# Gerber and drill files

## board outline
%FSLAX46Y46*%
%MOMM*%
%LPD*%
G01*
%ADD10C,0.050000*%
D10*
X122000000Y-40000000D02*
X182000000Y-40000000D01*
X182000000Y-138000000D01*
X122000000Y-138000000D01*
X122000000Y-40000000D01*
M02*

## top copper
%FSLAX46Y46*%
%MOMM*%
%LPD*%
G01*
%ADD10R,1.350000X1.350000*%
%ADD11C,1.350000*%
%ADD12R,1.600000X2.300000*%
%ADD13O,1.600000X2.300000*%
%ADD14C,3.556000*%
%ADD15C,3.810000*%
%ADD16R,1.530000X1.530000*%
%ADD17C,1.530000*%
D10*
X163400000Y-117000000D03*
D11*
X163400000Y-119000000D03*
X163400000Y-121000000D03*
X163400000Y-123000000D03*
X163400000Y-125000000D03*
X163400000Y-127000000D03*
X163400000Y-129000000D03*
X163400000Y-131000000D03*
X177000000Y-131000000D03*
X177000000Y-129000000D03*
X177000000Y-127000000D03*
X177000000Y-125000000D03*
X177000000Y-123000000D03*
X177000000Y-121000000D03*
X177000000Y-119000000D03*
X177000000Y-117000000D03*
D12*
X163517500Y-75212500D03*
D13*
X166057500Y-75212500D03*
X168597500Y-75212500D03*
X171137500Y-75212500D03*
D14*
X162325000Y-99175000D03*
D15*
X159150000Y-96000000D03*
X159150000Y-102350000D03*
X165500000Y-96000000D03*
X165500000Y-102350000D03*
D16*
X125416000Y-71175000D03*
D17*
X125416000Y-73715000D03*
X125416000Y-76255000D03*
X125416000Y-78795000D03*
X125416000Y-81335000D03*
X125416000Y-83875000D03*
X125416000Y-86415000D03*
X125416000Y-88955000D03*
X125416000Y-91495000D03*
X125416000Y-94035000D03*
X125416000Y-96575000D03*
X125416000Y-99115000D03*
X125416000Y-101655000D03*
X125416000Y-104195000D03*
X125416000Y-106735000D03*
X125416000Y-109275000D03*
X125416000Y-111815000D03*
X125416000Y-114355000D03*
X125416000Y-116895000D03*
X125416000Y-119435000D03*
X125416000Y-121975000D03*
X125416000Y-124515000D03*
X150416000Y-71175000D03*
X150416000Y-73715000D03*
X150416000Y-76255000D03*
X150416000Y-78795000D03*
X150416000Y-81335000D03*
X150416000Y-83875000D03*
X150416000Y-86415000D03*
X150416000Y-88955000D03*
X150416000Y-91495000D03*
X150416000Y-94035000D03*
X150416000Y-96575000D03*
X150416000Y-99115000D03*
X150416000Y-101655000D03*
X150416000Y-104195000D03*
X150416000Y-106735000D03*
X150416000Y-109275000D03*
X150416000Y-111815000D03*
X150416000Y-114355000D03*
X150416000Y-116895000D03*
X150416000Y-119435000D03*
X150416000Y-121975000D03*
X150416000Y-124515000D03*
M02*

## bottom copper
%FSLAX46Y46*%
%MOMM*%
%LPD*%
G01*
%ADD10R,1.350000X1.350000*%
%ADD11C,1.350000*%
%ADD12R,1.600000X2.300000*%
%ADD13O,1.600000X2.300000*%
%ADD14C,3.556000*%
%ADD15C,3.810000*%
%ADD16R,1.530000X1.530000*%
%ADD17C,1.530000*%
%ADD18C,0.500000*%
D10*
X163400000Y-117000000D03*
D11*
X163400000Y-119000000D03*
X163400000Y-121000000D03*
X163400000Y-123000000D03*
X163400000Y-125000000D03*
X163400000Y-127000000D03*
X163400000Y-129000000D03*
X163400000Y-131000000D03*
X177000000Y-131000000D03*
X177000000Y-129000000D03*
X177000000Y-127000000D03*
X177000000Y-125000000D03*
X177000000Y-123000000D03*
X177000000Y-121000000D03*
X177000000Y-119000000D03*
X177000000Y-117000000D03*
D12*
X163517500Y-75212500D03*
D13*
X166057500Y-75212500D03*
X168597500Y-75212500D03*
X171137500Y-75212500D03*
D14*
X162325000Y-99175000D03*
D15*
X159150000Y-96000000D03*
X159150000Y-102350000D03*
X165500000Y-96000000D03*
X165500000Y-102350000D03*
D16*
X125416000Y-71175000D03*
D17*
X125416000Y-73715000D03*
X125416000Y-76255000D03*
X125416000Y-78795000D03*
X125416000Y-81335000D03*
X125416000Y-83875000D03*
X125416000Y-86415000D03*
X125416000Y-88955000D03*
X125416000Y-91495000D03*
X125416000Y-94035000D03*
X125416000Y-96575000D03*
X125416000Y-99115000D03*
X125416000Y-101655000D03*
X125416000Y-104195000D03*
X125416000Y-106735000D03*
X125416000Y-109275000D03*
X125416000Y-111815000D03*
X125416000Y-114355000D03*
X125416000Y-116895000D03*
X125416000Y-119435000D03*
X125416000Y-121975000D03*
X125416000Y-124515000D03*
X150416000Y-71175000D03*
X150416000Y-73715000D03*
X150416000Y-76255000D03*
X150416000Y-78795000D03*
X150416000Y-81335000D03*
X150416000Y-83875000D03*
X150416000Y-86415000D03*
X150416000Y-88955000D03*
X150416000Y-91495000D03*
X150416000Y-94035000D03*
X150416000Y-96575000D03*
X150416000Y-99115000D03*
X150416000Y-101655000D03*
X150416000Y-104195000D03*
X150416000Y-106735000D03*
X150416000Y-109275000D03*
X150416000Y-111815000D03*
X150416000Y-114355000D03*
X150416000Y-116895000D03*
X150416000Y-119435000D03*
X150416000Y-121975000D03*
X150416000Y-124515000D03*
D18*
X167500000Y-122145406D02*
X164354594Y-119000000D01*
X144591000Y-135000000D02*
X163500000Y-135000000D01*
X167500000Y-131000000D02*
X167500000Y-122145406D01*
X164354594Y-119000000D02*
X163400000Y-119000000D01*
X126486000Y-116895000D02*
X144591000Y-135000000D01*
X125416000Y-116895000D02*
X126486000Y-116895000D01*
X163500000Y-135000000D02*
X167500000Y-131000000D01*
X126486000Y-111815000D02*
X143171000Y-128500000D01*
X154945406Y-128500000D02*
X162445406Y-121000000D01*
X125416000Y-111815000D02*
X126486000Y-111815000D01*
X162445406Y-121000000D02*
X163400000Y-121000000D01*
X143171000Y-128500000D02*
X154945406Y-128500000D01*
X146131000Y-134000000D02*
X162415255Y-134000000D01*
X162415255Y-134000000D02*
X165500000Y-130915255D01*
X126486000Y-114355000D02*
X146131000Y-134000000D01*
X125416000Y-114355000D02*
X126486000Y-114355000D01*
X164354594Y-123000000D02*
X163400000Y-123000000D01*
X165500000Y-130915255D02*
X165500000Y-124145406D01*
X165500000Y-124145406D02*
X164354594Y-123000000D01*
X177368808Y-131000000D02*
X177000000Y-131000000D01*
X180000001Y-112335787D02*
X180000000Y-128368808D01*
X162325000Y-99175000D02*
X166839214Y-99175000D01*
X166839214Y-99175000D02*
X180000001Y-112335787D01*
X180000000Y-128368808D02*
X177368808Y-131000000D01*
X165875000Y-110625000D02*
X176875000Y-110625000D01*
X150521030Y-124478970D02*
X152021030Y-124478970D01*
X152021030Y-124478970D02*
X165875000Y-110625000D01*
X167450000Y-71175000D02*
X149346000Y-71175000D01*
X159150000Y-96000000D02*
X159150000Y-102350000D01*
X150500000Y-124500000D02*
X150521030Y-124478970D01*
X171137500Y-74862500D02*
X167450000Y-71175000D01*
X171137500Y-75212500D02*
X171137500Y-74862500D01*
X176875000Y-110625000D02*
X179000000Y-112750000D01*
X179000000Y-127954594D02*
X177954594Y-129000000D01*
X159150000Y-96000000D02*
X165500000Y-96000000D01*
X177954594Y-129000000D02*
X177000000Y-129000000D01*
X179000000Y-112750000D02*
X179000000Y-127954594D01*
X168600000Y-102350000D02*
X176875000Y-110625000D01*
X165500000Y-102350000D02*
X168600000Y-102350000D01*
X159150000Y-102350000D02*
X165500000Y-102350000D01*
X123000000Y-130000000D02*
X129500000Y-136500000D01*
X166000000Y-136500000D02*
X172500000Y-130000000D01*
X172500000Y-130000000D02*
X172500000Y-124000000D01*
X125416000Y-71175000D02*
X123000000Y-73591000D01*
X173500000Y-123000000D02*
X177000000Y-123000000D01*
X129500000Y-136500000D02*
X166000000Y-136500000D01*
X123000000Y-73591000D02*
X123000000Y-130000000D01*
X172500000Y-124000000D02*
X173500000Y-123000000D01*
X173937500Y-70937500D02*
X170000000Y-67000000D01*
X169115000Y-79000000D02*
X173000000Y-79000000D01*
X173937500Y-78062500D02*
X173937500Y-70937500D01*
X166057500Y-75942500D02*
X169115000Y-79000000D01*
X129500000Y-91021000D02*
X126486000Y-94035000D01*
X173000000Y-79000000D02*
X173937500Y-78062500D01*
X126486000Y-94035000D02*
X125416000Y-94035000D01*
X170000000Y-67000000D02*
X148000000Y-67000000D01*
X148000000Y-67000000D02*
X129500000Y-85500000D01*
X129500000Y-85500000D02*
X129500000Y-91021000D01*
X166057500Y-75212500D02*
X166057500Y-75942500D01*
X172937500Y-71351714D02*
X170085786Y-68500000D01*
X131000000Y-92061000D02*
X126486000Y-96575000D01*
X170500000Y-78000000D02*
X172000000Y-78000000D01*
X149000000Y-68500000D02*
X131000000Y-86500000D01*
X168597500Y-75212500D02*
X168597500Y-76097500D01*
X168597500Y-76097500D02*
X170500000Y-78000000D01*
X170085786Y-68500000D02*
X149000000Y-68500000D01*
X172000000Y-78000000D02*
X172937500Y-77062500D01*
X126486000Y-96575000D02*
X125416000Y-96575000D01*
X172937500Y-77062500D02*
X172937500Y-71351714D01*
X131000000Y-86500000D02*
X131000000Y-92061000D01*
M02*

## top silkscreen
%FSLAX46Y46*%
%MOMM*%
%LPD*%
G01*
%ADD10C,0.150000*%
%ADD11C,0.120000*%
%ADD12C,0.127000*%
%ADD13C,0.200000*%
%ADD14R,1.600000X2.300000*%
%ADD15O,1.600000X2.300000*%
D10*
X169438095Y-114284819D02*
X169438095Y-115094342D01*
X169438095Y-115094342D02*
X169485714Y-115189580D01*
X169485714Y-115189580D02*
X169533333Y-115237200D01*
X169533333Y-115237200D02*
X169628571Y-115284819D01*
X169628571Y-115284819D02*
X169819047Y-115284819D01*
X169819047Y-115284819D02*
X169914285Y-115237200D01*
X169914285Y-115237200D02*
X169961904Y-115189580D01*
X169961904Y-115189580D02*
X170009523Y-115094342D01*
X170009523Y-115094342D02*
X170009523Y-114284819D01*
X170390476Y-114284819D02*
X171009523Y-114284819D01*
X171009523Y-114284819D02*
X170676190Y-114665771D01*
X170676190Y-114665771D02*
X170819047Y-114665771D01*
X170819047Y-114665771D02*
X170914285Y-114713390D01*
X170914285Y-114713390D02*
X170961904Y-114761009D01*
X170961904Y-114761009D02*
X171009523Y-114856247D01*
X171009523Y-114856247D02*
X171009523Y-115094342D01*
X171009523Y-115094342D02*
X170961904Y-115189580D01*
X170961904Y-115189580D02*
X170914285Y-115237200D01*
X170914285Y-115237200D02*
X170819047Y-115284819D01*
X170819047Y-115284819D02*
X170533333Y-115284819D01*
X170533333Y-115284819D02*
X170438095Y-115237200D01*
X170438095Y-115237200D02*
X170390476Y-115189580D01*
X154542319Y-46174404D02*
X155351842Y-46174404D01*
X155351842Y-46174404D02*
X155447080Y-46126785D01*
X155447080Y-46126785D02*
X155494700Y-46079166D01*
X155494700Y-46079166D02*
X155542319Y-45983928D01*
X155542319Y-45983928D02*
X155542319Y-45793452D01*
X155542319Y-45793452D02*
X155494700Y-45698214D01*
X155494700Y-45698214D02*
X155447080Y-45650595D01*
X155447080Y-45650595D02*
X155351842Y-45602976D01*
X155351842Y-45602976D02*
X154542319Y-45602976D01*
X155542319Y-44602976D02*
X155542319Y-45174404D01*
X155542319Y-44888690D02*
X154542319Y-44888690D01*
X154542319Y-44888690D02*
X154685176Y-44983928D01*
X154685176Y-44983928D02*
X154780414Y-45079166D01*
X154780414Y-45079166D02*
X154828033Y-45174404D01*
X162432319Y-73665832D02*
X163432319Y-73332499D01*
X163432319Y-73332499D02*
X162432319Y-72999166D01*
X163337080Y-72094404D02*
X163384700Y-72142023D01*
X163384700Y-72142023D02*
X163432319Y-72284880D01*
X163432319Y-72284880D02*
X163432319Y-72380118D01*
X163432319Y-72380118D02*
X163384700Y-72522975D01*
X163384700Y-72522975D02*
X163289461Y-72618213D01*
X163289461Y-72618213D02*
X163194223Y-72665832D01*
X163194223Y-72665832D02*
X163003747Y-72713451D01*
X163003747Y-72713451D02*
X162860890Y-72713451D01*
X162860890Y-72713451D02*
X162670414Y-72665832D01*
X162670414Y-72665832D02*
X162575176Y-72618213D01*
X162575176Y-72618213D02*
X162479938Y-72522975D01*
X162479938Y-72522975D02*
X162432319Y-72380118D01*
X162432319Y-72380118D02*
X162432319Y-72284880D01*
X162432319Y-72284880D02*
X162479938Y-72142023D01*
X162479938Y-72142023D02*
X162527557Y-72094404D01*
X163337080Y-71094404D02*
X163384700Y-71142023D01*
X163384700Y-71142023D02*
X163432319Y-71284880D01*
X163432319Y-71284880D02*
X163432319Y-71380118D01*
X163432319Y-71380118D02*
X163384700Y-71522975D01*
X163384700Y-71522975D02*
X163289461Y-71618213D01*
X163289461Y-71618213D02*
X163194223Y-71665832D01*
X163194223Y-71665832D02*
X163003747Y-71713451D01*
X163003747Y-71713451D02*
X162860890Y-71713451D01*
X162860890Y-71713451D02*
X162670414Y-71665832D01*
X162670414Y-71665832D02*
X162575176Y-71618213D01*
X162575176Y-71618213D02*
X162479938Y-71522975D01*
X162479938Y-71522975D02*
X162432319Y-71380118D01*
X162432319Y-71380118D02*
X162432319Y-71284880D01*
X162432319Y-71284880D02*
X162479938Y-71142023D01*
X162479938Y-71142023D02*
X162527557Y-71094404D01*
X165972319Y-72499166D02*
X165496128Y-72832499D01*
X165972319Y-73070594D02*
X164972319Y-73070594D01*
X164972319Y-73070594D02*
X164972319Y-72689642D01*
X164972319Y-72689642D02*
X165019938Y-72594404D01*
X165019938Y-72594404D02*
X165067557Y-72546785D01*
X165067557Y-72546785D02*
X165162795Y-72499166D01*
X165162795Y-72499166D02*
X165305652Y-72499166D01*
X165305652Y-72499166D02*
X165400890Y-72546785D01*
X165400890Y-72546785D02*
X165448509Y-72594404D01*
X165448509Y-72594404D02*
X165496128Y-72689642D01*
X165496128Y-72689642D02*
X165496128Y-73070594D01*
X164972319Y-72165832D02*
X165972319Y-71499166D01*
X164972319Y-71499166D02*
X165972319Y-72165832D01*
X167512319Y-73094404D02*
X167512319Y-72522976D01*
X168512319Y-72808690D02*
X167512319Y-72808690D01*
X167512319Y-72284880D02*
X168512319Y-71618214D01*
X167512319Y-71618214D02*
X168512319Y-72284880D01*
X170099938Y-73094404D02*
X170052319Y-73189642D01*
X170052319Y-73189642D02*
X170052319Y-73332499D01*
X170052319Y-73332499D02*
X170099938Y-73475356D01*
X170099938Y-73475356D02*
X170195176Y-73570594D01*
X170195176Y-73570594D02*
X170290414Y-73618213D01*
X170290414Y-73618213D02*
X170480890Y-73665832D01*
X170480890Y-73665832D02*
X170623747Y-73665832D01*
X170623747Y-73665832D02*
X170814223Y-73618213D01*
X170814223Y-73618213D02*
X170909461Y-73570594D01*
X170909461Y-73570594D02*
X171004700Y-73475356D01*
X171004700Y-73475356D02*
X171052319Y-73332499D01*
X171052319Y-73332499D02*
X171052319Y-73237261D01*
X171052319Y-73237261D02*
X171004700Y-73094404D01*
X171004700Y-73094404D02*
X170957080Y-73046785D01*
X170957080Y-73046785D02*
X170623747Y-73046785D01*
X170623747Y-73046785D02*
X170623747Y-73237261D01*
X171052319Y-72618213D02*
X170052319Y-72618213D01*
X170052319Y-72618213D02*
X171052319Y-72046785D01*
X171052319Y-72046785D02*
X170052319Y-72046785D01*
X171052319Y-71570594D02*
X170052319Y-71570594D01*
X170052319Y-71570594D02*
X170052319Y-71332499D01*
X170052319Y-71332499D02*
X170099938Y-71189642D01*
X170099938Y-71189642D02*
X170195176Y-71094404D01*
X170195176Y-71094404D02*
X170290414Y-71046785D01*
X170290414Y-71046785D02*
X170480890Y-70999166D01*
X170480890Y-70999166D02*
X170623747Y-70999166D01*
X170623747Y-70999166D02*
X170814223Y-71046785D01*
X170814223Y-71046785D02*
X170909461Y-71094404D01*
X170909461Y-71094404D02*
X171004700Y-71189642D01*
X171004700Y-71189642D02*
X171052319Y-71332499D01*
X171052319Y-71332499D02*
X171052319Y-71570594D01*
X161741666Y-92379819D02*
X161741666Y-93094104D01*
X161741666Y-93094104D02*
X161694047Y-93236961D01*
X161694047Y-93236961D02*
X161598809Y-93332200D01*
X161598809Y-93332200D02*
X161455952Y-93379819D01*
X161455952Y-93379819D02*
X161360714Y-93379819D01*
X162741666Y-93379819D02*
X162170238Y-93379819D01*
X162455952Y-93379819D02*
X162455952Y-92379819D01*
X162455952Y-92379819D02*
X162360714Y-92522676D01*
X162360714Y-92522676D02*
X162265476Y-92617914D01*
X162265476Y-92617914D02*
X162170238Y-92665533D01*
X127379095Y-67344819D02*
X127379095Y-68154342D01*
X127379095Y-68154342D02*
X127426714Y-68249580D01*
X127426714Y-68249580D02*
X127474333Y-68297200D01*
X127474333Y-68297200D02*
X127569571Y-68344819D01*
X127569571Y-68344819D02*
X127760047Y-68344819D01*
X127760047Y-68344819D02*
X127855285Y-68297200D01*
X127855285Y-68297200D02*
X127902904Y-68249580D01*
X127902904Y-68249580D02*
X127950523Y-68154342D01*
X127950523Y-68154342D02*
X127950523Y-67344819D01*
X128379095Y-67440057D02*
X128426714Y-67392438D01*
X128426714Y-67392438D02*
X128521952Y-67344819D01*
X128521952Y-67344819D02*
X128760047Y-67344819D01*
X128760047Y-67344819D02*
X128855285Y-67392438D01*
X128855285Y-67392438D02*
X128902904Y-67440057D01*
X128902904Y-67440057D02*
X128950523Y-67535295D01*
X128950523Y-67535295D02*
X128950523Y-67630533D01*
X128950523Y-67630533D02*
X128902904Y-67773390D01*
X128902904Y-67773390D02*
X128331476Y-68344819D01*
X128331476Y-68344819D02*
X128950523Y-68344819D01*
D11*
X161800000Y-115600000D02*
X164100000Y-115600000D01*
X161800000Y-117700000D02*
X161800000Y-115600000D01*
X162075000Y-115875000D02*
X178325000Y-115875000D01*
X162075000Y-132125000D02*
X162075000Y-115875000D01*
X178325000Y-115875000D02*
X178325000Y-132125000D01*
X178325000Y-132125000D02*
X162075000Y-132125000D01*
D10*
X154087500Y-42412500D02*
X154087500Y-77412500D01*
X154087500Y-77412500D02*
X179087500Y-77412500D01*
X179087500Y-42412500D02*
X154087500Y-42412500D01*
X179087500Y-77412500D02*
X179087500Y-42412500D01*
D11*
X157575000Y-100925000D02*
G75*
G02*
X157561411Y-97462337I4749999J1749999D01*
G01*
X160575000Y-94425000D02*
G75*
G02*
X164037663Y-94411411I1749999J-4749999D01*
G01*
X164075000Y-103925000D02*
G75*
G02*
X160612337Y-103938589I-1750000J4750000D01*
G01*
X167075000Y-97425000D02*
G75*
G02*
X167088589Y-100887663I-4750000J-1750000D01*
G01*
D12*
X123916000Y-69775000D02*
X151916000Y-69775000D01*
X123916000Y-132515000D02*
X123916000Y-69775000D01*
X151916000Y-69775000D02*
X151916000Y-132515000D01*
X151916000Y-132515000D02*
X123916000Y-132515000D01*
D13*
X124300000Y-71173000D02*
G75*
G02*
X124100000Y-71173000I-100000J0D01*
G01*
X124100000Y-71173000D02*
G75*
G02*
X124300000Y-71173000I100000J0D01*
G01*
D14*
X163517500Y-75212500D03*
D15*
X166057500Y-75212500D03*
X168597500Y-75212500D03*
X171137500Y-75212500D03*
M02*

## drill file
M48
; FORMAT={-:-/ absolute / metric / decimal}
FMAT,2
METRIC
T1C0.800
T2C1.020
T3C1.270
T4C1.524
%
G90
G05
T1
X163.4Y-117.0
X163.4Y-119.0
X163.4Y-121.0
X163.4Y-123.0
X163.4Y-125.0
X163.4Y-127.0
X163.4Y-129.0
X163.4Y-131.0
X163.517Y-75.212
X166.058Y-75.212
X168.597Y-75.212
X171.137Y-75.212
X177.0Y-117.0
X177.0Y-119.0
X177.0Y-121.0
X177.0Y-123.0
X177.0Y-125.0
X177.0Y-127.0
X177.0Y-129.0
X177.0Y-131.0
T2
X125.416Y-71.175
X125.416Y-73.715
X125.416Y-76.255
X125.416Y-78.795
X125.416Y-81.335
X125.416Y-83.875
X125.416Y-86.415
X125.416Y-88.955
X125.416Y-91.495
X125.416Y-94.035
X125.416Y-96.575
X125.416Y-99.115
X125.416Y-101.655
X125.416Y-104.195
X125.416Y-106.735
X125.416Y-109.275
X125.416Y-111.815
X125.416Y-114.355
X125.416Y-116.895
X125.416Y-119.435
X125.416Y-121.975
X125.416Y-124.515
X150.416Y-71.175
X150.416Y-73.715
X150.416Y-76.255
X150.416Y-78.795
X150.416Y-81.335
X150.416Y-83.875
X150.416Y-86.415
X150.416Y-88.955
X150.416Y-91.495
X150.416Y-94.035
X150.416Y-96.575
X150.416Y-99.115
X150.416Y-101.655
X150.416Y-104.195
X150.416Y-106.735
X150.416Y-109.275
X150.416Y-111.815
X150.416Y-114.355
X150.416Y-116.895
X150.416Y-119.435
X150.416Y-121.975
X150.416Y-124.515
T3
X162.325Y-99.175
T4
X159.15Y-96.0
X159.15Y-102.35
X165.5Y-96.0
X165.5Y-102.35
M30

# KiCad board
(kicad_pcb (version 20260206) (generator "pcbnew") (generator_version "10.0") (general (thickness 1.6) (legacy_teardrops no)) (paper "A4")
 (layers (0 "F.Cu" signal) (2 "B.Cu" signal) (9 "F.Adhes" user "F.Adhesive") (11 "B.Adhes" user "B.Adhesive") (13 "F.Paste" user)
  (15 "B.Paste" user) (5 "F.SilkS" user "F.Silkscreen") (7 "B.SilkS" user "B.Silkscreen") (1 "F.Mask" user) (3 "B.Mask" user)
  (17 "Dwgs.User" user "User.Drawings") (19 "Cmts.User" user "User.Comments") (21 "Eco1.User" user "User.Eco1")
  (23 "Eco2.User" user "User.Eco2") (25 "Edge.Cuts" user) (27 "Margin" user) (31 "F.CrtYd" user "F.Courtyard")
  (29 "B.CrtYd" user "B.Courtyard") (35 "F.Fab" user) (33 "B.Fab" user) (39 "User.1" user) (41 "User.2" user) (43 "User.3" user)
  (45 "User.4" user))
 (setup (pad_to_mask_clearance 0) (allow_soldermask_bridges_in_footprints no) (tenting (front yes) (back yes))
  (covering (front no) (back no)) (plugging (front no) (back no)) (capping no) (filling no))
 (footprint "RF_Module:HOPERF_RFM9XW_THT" (layer "F.Cu") (at 163.4 117)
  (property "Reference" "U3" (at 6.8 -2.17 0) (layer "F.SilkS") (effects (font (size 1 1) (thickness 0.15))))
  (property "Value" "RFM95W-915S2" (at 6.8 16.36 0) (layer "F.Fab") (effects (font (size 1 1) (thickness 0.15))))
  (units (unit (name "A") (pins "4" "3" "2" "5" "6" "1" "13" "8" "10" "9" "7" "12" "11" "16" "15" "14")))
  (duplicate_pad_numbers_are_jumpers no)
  (fp_line (start -1.6 -1.4) (end 0.7 -1.4) (stroke (width 0.12) (type solid)) (layer "F.SilkS"))
  (fp_line (start -1.6 0.7) (end -1.6 -1.4) (stroke (width 0.12) (type solid)) (layer "F.SilkS"))
  (fp_line (start -1.325 -1.125) (end 14.925 -1.125) (stroke (width 0.12) (type solid)) (layer "F.SilkS"))
  (fp_line (start -1.325 15.125) (end -1.325 -1.125) (stroke (width 0.12) (type solid)) (layer "F.SilkS"))
  (fp_line (start 14.925 -1.125) (end 14.925 15.125) (stroke (width 0.12) (type solid)) (layer "F.SilkS"))
  (fp_line (start 14.925 15.125) (end -1.325 15.125) (stroke (width 0.12) (type solid)) (layer "F.SilkS"))
  (pad "1" thru_hole rect (at 0 0) (size 1.35 1.35) (drill 0.8) (layers "*.Cu" "*.Mask") (remove_unused_layers no)
   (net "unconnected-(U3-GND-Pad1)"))
  (pad "2" thru_hole circle (at 0 2) (size 1.35 1.35) (drill 0.8) (layers "*.Cu" "*.Mask") (remove_unused_layers no) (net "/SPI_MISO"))
  (pad "3" thru_hole circle (at 0 4) (size 1.35 1.35) (drill 0.8) (layers "*.Cu" "*.Mask") (remove_unused_layers no) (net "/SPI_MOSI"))
  (pad "4" thru_hole circle (at 0 6) (size 1.35 1.35) (drill 0.8) (layers "*.Cu" "*.Mask") (remove_unused_layers no) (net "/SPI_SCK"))
  (pad "5" thru_hole circle (at 0 8) (size 1.35 1.35) (drill 0.8) (layers "*.Cu" "*.Mask") (remove_unused_layers no) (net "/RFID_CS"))
  (pad "6" thru_hole circle (at 0 10) (size 1.35 1.35) (drill 0.8) (layers "*.Cu" "*.Mask") (remove_unused_layers no) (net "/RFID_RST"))
  (pad "7" thru_hole circle (at 0 12) (size 1.35 1.35) (drill 0.8) (layers "*.Cu" "*.Mask") (remove_unused_layers no)
   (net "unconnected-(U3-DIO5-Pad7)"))
  (pad "8" thru_hole circle (at 0 14) (size 1.35 1.35) (drill 0.8) (layers "*.Cu" "*.Mask") (remove_unused_layers no)
   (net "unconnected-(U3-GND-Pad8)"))
  (pad "9" thru_hole circle (at 13.6 14) (size 1.35 1.35) (drill 0.8) (layers "*.Cu" "*.Mask") (remove_unused_layers no) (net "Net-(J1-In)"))
  (pad "10" thru_hole circle (at 13.6 12) (size 1.35 1.35) (drill 0.8) (layers "*.Cu" "*.Mask") (remove_unused_layers no)
   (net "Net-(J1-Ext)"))
  (pad "11" thru_hole circle (at 13.6 10) (size 1.35 1.35) (drill 0.8) (layers "*.Cu" "*.Mask") (remove_unused_layers no)
   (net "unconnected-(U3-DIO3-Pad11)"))
  (pad "12" thru_hole circle (at 13.6 8) (size 1.35 1.35) (drill 0.8) (layers "*.Cu" "*.Mask") (remove_unused_layers no)
   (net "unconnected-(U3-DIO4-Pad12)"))
  (pad "13" thru_hole circle (at 13.6 6) (size 1.35 1.35) (drill 0.8) (layers "*.Cu" "*.Mask") (remove_unused_layers no)
   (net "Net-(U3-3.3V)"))
  (pad "14" thru_hole circle (at 13.6 4) (size 1.35 1.35) (drill 0.8) (layers "*.Cu" "*.Mask") (remove_unused_layers no)
   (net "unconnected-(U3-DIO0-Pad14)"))
  (pad "15" thru_hole circle (at 13.6 2) (size 1.35 1.35) (drill 0.8) (layers "*.Cu" "*.Mask") (remove_unused_layers no)
   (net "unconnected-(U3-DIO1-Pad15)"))
  (pad "16" thru_hole circle (at 13.6 0) (size 1.35 1.35) (drill 0.8) (layers "*.Cu" "*.Mask") (remove_unused_layers no)
   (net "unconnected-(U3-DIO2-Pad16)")))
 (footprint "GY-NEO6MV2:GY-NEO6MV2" (layer "F.Cu") (at 154.0875 77.4125 -90)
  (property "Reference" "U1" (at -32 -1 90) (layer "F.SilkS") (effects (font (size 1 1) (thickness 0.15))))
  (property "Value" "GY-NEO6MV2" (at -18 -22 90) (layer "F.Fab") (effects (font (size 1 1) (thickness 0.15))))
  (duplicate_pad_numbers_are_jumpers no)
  (fp_line (start -35 0) (end 0 0) (stroke (width 0.15) (type solid)) (layer "F.SilkS"))
  (fp_line (start 0 0) (end 0 -25) (stroke (width 0.15) (type solid)) (layer "F.SilkS"))
  (fp_line (start -35 -25) (end -35 0) (stroke (width 0.15) (type solid)) (layer "F.SilkS"))
  (fp_line (start 0 -25) (end -35 -25) (stroke (width 0.15) (type solid)) (layer "F.SilkS"))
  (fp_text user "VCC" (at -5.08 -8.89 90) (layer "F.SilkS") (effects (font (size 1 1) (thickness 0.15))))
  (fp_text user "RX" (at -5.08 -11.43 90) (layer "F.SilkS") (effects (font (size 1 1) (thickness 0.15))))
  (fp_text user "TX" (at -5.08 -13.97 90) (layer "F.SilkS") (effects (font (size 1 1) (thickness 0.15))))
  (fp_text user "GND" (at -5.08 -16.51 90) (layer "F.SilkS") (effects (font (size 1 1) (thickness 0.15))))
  (pad "1" thru_hole rect (at -2.2 -9.43 270) (size 2.3 1.6) (drill 0.8) (layers "*.Cu" "*.Mask" "F.SilkS") (remove_unused_layers no)
   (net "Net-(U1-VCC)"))
  (pad "2" thru_hole oval (at -2.2 -11.97 270) (size 2.3 1.6) (drill 0.8) (layers "*.Cu" "*.Mask" "F.SilkS") (remove_unused_layers no)
   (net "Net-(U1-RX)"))
  (pad "3" thru_hole oval (at -2.2 -14.51 270) (size 2.3 1.6) (drill 0.8) (layers "*.Cu" "*.Mask" "F.SilkS") (remove_unused_layers no)
   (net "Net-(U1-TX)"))
  (pad "4" thru_hole oval (at -2.2 -17.05 270) (size 2.3 1.6) (drill 0.8) (layers "*.Cu" "*.Mask" "F.SilkS") (remove_unused_layers no)
   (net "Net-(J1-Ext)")))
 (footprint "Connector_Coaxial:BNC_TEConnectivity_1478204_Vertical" (layer "F.Cu") (at 162.325 99.175)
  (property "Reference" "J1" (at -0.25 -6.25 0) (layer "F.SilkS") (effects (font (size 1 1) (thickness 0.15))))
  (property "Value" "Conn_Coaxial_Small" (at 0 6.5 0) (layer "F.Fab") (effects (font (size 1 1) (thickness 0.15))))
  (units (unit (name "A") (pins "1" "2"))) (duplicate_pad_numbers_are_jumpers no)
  (fp_arc (start -4.75 1.75) (mid -5.062075 0.019867) (end -4.763589 -1.712663) (stroke (width 0.12) (type solid)) (layer "F.SilkS"))
  (fp_arc (start -1.75 -4.75) (mid -0.019867 -5.062075) (end 1.712663 -4.763589) (stroke (width 0.12) (type solid)) (layer "F.SilkS"))
  (fp_arc (start 1.75 4.75) (mid 0.019867 5.062075) (end -1.712663 4.763589) (stroke (width 0.12) (type solid)) (layer "F.SilkS"))
  (fp_arc (start 4.75 -1.75) (mid 5.062075 -0.019867) (end 4.763589 1.712663) (stroke (width 0.12) (type solid)) (layer "F.SilkS"))
  (pad "1" thru_hole circle (at 0 0) (size 3.556 3.556) (drill 1.27) (layers "*.Cu" "*.Mask") (remove_unused_layers no) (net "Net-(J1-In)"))
  (pad "2" thru_hole circle (at -3.175 -3.175) (size 3.81 3.81) (drill 1.524) (layers "*.Cu" "*.Mask") (remove_unused_layers no)
   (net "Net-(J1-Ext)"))
  (pad "2" thru_hole circle (at -3.175 3.175) (size 3.81 3.81) (drill 1.524) (layers "*.Cu" "*.Mask") (remove_unused_layers no)
   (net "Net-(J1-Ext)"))
  (pad "2" thru_hole circle (at 3.175 -3.175) (size 3.81 3.81) (drill 1.524) (layers "*.Cu" "*.Mask") (remove_unused_layers no)
   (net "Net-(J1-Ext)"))
  (pad "2" thru_hole circle (at 3.175 3.175) (size 3.81 3.81) (drill 1.524) (layers "*.Cu" "*.Mask") (remove_unused_layers no)
   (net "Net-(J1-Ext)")))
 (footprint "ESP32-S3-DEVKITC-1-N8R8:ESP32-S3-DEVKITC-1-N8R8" (layer "F.Cu") (at 137.916 101.145)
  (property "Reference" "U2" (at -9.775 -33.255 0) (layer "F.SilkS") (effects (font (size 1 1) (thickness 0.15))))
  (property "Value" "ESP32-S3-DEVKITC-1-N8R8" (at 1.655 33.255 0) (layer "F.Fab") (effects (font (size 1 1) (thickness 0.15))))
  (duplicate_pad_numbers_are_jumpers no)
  (fp_line (start -14 -31.37) (end 14 -31.37) (stroke (width 0.127) (type solid)) (layer "F.SilkS"))
  (fp_line (start -14 31.37) (end -14 -31.37) (stroke (width 0.127) (type solid)) (layer "F.SilkS"))
  (fp_line (start 14 -31.37) (end 14 31.37) (stroke (width 0.127) (type solid)) (layer "F.SilkS"))
  (fp_line (start 14 31.37) (end -14 31.37) (stroke (width 0.127) (type solid)) (layer "F.SilkS"))
  (fp_circle (center -13.716 -29.972) (end -13.616 -29.972) (stroke (width 0.2) (type solid)) (fill no) (layer "F.SilkS"))
  (pad "J1_1" thru_hole rect (at -12.5 -29.97) (size 1.53 1.53) (drill 1.02) (layers "*.Cu" "*.Mask") (remove_unused_layers no)
   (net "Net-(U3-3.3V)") (solder_mask_margin 0.102))
  (pad "J1_2" thru_hole circle (at -12.5 -27.43) (size 1.53 1.53) (drill 1.02) (layers "*.Cu" "*.Mask") (remove_unused_layers no)
   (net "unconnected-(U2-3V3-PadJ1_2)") (solder_mask_margin 0.102))
  (pad "J1_3" thru_hole circle (at -12.5 -24.89) (size 1.53 1.53) (drill 1.02) (layers "*.Cu" "*.Mask") (remove_unused_layers no)
   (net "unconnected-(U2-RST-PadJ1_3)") (solder_mask_margin 0.102))
  (pad "J1_4" thru_hole circle (at -12.5 -22.35) (size 1.53 1.53) (drill 1.02) (layers "*.Cu" "*.Mask") (remove_unused_layers no)
   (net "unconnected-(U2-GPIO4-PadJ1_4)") (solder_mask_margin 0.102))
  (pad "J1_5" thru_hole circle (at -12.5 -19.81) (size 1.53 1.53) (drill 1.02) (layers "*.Cu" "*.Mask") (remove_unused_layers no)
   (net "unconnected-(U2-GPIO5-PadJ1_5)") (solder_mask_margin 0.102))
  (pad "J1_6" thru_hole circle (at -12.5 -17.27) (size 1.53 1.53) (drill 1.02) (layers "*.Cu" "*.Mask") (remove_unused_layers no)
   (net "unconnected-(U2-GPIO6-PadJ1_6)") (solder_mask_margin 0.102))
  (pad "J1_7" thru_hole circle (at -12.5 -14.73) (size 1.53 1.53) (drill 1.02) (layers "*.Cu" "*.Mask") (remove_unused_layers no)
   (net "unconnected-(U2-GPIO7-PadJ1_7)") (solder_mask_margin 0.102))
  (pad "J1_8" thru_hole circle (at -12.5 -12.19) (size 1.53 1.53) (drill 1.02) (layers "*.Cu" "*.Mask") (remove_unused_layers no)
   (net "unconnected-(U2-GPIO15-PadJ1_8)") (solder_mask_margin 0.102))
  (pad "J1_9" thru_hole circle (at -12.5 -9.65) (size 1.53 1.53) (drill 1.02) (layers "*.Cu" "*.Mask") (remove_unused_layers no)
   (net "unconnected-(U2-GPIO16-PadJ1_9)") (solder_mask_margin 0.102))
  (pad "J1_10" thru_hole circle (at -12.5 -7.11) (size 1.53 1.53) (drill 1.02) (layers "*.Cu" "*.Mask") (remove_unused_layers no)
   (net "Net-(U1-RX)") (solder_mask_margin 0.102))
  (pad "J1_11" thru_hole circle (at -12.5 -4.57) (size 1.53 1.53) (drill 1.02) (layers "*.Cu" "*.Mask") (remove_unused_layers no)
   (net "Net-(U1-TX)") (solder_mask_margin 0.102))
  (pad "J1_12" thru_hole circle (at -12.5 -2.03) (size 1.53 1.53) (drill 1.02) (layers "*.Cu" "*.Mask") (remove_unused_layers no)
   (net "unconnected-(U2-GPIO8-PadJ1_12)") (solder_mask_margin 0.102))
  (pad "J1_13" thru_hole circle (at -12.5 0.51) (size 1.53 1.53) (drill 1.02) (layers "*.Cu" "*.Mask") (remove_unused_layers no)
   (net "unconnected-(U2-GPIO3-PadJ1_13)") (solder_mask_margin 0.102))
  (pad "J1_14" thru_hole circle (at -12.5 3.05) (size 1.53 1.53) (drill 1.02) (layers "*.Cu" "*.Mask") (remove_unused_layers no)
   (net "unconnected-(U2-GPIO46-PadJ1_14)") (solder_mask_margin 0.102))
  (pad "J1_15" thru_hole circle (at -12.5 5.59) (size 1.53 1.53) (drill 1.02) (layers "*.Cu" "*.Mask") (remove_unused_layers no)
   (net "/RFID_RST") (solder_mask_margin 0.102))
  (pad "J1_16" thru_hole circle (at -12.5 8.13) (size 1.53 1.53) (drill 1.02) (layers "*.Cu" "*.Mask") (remove_unused_layers no)
   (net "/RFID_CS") (solder_mask_margin 0.102))
  (pad "J1_17" thru_hole circle (at -12.5 10.67) (size 1.53 1.53) (drill 1.02) (layers "*.Cu" "*.Mask") (remove_unused_layers no)
   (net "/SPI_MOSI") (solder_mask_margin 0.102))
  (pad "J1_18" thru_hole circle (at -12.5 13.21) (size 1.53 1.53) (drill 1.02) (layers "*.Cu" "*.Mask") (remove_unused_layers no)
   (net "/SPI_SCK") (solder_mask_margin 0.102))
  (pad "J1_19" thru_hole circle (at -12.5 15.75) (size 1.53 1.53) (drill 1.02) (layers "*.Cu" "*.Mask") (remove_unused_layers no)
   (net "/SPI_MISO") (solder_mask_margin 0.102))
  (pad "J1_20" thru_hole circle (at -12.5 18.29) (size 1.53 1.53) (drill 1.02) (layers "*.Cu" "*.Mask") (remove_unused_layers no)
   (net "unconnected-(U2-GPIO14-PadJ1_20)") (solder_mask_margin 0.102))
  (pad "J1_21" thru_hole circle (at -12.5 20.83) (size 1.53 1.53) (drill 1.02) (layers "*.Cu" "*.Mask") (remove_unused_layers no)
   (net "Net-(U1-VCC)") (solder_mask_margin 0.102))
  (pad "J1_22" thru_hole circle (at -12.5 23.37) (size 1.53 1.53) (drill 1.02) (layers "*.Cu" "*.Mask") (remove_unused_layers no)
   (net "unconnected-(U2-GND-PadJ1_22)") (solder_mask_margin 0.102))
  (pad "J3_1" thru_hole circle (at 12.5 -29.97) (size 1.53 1.53) (drill 1.02) (layers "*.Cu" "*.Mask") (remove_unused_layers no)
   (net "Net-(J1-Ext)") (solder_mask_margin 0.102))
  (pad "J3_2" thru_hole circle (at 12.5 -27.43) (size 1.53 1.53) (drill 1.02) (layers "*.Cu" "*.Mask") (remove_unused_layers no)
   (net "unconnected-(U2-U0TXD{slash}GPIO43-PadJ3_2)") (solder_mask_margin 0.102))
  (pad "J3_3" thru_hole circle (at 12.5 -24.89) (size 1.53 1.53) (drill 1.02) (layers "*.Cu" "*.Mask") (remove_unused_layers no)
   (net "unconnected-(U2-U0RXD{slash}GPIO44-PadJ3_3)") (solder_mask_margin 0.102))
  (pad "J3_4" thru_hole circle (at 12.5 -22.35) (size 1.53 1.53) (drill 1.02) (layers "*.Cu" "*.Mask") (remove_unused_layers no)
   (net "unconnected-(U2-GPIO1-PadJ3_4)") (solder_mask_margin 0.102))
  (pad "J3_5" thru_hole circle (at 12.5 -19.81) (size 1.53 1.53) (drill 1.02) (layers "*.Cu" "*.Mask") (remove_unused_layers no)
   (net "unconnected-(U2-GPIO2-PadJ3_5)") (solder_mask_margin 0.102))
  (pad "J3_6" thru_hole circle (at 12.5 -17.27) (size 1.53 1.53) (drill 1.02) (layers "*.Cu" "*.Mask") (remove_unused_layers no)
   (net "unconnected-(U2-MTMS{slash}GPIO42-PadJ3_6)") (solder_mask_margin 0.102))
  (pad "J3_7" thru_hole circle (at 12.5 -14.73) (size 1.53 1.53) (drill 1.02) (layers "*.Cu" "*.Mask") (remove_unused_layers no)
   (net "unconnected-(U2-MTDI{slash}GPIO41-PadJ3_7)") (solder_mask_margin 0.102))
  (pad "J3_8" thru_hole circle (at 12.5 -12.19) (size 1.53 1.53) (drill 1.02) (layers "*.Cu" "*.Mask") (remove_unused_layers no)
   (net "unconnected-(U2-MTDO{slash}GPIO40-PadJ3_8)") (solder_mask_margin 0.102))
  (pad "J3_9" thru_hole circle (at 12.5 -9.65) (size 1.53 1.53) (drill 1.02) (layers "*.Cu" "*.Mask") (remove_unused_layers no)
   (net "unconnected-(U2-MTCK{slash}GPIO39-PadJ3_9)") (solder_mask_margin 0.102))
  (pad "J3_10" thru_hole circle (at 12.5 -7.11) (size 1.53 1.53) (drill 1.02) (layers "*.Cu" "*.Mask") (remove_unused_layers no)
   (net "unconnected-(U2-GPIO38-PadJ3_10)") (solder_mask_margin 0.102))
  (pad "J3_11" thru_hole circle (at 12.5 -4.57) (size 1.53 1.53) (drill 1.02) (layers "*.Cu" "*.Mask") (remove_unused_layers no)
   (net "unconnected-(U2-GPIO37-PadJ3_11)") (solder_mask_margin 0.102))
  (pad "J3_12" thru_hole circle (at 12.5 -2.03) (size 1.53 1.53) (drill 1.02) (layers "*.Cu" "*.Mask") (remove_unused_layers no)
   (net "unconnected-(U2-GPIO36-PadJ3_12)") (solder_mask_margin 0.102))
  (pad "J3_13" thru_hole circle (at 12.5 0.51) (size 1.53 1.53) (drill 1.02) (layers "*.Cu" "*.Mask") (remove_unused_layers no)
   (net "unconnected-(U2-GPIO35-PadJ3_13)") (solder_mask_margin 0.102))
  (pad "J3_14" thru_hole circle (at 12.5 3.05) (size 1.53 1.53) (drill 1.02) (layers "*.Cu" "*.Mask") (remove_unused_layers no)
   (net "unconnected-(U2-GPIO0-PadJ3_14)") (solder_mask_margin 0.102))
  (pad "J3_15" thru_hole circle (at 12.5 5.59) (size 1.53 1.53) (drill 1.02) (layers "*.Cu" "*.Mask") (remove_unused_layers no)
   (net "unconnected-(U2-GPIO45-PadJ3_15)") (solder_mask_margin 0.102))
  (pad "J3_16" thru_hole circle (at 12.5 8.13) (size 1.53 1.53) (drill 1.02) (layers "*.Cu" "*.Mask") (remove_unused_layers no)
   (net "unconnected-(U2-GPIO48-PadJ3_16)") (solder_mask_margin 0.102))
  (pad "J3_17" thru_hole circle (at 12.5 10.67) (size 1.53 1.53) (drill 1.02) (layers "*.Cu" "*.Mask") (remove_unused_layers no)
   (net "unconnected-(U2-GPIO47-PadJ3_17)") (solder_mask_margin 0.102))
  (pad "J3_18" thru_hole circle (at 12.5 13.21) (size 1.53 1.53) (drill 1.02) (layers "*.Cu" "*.Mask") (remove_unused_layers no)
   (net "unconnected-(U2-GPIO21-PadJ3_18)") (solder_mask_margin 0.102))
  (pad "J3_19" thru_hole circle (at 12.5 15.75) (size 1.53 1.53) (drill 1.02) (layers "*.Cu" "*.Mask") (remove_unused_layers no)
   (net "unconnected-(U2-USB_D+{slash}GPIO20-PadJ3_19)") (solder_mask_margin 0.102))
  (pad "J3_20" thru_hole circle (at 12.5 18.29) (size 1.53 1.53) (drill 1.02) (layers "*.Cu" "*.Mask") (remove_unused_layers no)
   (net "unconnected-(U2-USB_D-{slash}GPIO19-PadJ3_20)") (solder_mask_margin 0.102))
  (pad "J3_21" thru_hole circle (at 12.5 20.83) (size 1.53 1.53) (drill 1.02) (layers "*.Cu" "*.Mask") (remove_unused_layers no)
   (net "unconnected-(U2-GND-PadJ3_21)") (solder_mask_margin 0.102))
  (pad "J3_22" thru_hole circle (at 12.5 23.37) (size 1.53 1.53) (drill 1.02) (layers "*.Cu" "*.Mask") (remove_unused_layers no)
   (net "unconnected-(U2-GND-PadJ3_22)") (solder_mask_margin 0.102)))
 (gr_rect (start 122 40) (end 182 138) (stroke (width 0.05) (type solid)) (fill no) (layer "Edge.Cuts"))
 (segment (start 167.5 122.145406) (end 164.354594 119) (width 0.5) (layer "B.Cu") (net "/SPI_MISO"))
 (segment (start 144.591 135) (end 163.5 135) (width 0.5) (layer "B.Cu") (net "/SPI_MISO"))
 (segment (start 167.5 131) (end 167.5 122.145406) (width 0.5) (layer "B.Cu") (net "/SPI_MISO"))
 (segment (start 164.354594 119) (end 163.4 119) (width 0.5) (layer "B.Cu") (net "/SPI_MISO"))
 (segment (start 126.486 116.895) (end 144.591 135) (width 0.5) (layer "B.Cu") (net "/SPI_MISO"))
 (segment (start 125.416 116.895) (end 126.486 116.895) (width 0.5) (layer "B.Cu") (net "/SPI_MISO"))
 (segment (start 163.5 135) (end 167.5 131) (width 0.5) (layer "B.Cu") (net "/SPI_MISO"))
 (segment (start 126.486 111.815) (end 143.171 128.5) (width 0.5) (layer "B.Cu") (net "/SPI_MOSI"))
 (segment (start 154.945406 128.5) (end 162.445406 121) (width 0.5) (layer "B.Cu") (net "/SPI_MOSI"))
 (segment (start 125.416 111.815) (end 126.486 111.815) (width 0.5) (layer "B.Cu") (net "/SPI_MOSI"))
 (segment (start 162.445406 121) (end 163.4 121) (width 0.5) (layer "B.Cu") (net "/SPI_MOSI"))
 (segment (start 143.171 128.5) (end 154.945406 128.5) (width 0.5) (layer "B.Cu") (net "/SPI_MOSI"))
 (segment (start 146.131 134) (end 162.415255 134) (width 0.5) (layer "B.Cu") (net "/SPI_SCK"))
 (segment (start 162.415255 134) (end 165.5 130.915255) (width 0.5) (layer "B.Cu") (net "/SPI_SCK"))
 (segment (start 126.486 114.355) (end 146.131 134) (width 0.5) (layer "B.Cu") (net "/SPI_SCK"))
 (segment (start 125.416 114.355) (end 126.486 114.355) (width 0.5) (layer "B.Cu") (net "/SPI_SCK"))
 (segment (start 164.354594 123) (end 163.4 123) (width 0.5) (layer "B.Cu") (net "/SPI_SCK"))
 (segment (start 165.5 130.915255) (end 165.5 124.145406) (width 0.5) (layer "B.Cu") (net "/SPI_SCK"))
 (segment (start 165.5 124.145406) (end 164.354594 123) (width 0.5) (layer "B.Cu") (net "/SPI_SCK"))
 (segment (start 177.368808 131) (end 177 131) (width 0.5) (layer "B.Cu") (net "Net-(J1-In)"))
 (segment (start 180.000001 112.335787) (end 180 128.368808) (width 0.5) (layer "B.Cu") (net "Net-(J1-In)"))
 (segment (start 162.325 99.175) (end 166.839214 99.175) (width 0.5) (layer "B.Cu") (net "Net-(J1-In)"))
 (segment (start 166.839214 99.175) (end 180.000001 112.335787) (width 0.5) (layer "B.Cu") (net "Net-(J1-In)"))
 (segment (start 180 128.368808) (end 177.368808 131) (width 0.5) (layer "B.Cu") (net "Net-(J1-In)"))
 (segment (start 165.875 110.625) (end 176.875 110.625) (width 0.5) (layer "B.Cu") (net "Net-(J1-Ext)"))
 (segment (start 150.52103 124.47897) (end 152.02103 124.47897) (width 0.5) (layer "B.Cu") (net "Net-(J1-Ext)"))
 (segment (start 152.02103 124.47897) (end 165.875 110.625) (width 0.5) (layer "B.Cu") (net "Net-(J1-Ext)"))
 (segment (start 167.45 71.175) (end 149.346 71.175) (width 0.5) (layer "B.Cu") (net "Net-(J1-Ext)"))
 (segment (start 159.15 96) (end 159.15 102.35) (width 0.5) (layer "B.Cu") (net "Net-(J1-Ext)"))
 (segment (start 150.5 124.5) (end 150.52103 124.47897) (width 0.5) (layer "B.Cu") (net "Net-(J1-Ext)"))
 (segment (start 171.1375 74.8625) (end 167.45 71.175) (width 0.5) (layer "B.Cu") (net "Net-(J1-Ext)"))
 (segment (start 171.1375 75.2125) (end 171.1375 74.8625) (width 0.5) (layer "B.Cu") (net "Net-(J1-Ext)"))
 (segment (start 176.875 110.625) (end 179 112.75) (width 0.5) (layer "B.Cu") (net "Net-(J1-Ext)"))
 (segment (start 179 127.954594) (end 177.954594 129) (width 0.5) (layer "B.Cu") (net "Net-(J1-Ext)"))
 (segment (start 159.15 96) (end 165.5 96) (width 0.5) (layer "B.Cu") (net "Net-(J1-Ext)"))
 (segment (start 177.954594 129) (end 177 129) (width 0.5) (layer "B.Cu") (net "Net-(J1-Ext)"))
 (segment (start 179 112.75) (end 179 127.954594) (width 0.5) (layer "B.Cu") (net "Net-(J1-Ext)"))
 (segment (start 168.6 102.35) (end 176.875 110.625) (width 0.5) (layer "B.Cu") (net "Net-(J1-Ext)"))
 (segment (start 165.5 102.35) (end 168.6 102.35) (width 0.5) (layer "B.Cu") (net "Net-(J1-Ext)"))
 (segment (start 159.15 102.35) (end 165.5 102.35) (width 0.5) (layer "B.Cu") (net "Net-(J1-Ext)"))
 (segment (start 123 130) (end 129.5 136.5) (width 0.5) (layer "B.Cu") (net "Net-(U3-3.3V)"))
 (segment (start 166 136.5) (end 172.5 130) (width 0.5) (layer "B.Cu") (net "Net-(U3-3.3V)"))
 (segment (start 172.5 130) (end 172.5 124) (width 0.5) (layer "B.Cu") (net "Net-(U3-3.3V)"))
 (segment (start 125.416 71.175) (end 123 73.591) (width 0.5) (layer "B.Cu") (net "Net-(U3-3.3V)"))
 (segment (start 173.5 123) (end 177 123) (width 0.5) (layer "B.Cu") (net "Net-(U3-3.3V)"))
 (segment (start 129.5 136.5) (end 166 136.5) (width 0.5) (layer "B.Cu") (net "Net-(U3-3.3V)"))
 (segment (start 123 73.591) (end 123 130) (width 0.5) (layer "B.Cu") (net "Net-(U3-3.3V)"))
 (segment (start 172.5 124) (end 173.5 123) (width 0.5) (layer "B.Cu") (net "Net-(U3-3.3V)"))
 (segment (start 173.9375 70.9375) (end 170 67) (width 0.5) (layer "B.Cu") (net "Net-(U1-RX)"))
 (segment (start 169.115 79) (end 173 79) (width 0.5) (layer "B.Cu") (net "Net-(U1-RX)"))
 (segment (start 173.9375 78.0625) (end 173.9375 70.9375) (width 0.5) (layer "B.Cu") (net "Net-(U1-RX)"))
 (segment (start 166.0575 75.9425) (end 169.115 79) (width 0.5) (layer "B.Cu") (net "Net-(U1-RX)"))
 (segment (start 129.5 91.021) (end 126.486 94.035) (width 0.5) (layer "B.Cu") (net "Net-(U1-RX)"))
 (segment (start 173 79) (end 173.9375 78.0625) (width 0.5) (layer "B.Cu") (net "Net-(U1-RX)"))
 (segment (start 126.486 94.035) (end 125.416 94.035) (width 0.5) (layer "B.Cu") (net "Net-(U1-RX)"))
 (segment (start 170 67) (end 148 67) (width 0.5) (layer "B.Cu") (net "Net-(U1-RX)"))
 (segment (start 148 67) (end 129.5 85.5) (width 0.5) (layer "B.Cu") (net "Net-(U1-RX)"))
 (segment (start 129.5 85.5) (end 129.5 91.021) (width 0.5) (layer "B.Cu") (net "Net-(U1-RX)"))
 (segment (start 166.0575 75.2125) (end 166.0575 75.9425) (width 0.5) (layer "B.Cu") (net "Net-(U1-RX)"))
 (segment (start 172.9375 71.351714) (end 170.085786 68.5) (width 0.5) (layer "B.Cu") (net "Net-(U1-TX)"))
 (segment (start 131 92.061) (end 126.486 96.575) (width 0.5) (layer "B.Cu") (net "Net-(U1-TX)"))
 (segment (start 170.5 78) (end 172 78) (width 0.5) (layer "B.Cu") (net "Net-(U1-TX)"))
 (segment (start 149 68.5) (end 131 86.5) (width 0.5) (layer "B.Cu") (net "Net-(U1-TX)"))
 (segment (start 168.5975 75.2125) (end 168.5975 76.0975) (width 0.5) (layer "B.Cu") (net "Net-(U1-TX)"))
 (segment (start 168.5975 76.0975) (end 170.5 78) (width 0.5) (layer "B.Cu") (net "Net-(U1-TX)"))
 (segment (start 170.085786 68.5) (end 149 68.5) (width 0.5) (layer "B.Cu") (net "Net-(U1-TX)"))
 (segment (start 172 78) (end 172.9375 77.0625) (width 0.5) (layer "B.Cu") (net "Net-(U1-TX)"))
 (segment (start 126.486 96.575) (end 125.416 96.575) (width 0.5) (layer "B.Cu") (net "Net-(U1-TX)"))
 (segment (start 172.9375 77.0625) (end 172.9375 71.351714) (width 0.5) (layer "B.Cu") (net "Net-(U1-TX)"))
 (segment (start 131 86.5) (end 131 92.061) (width 0.5) (layer "B.Cu") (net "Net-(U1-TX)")))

